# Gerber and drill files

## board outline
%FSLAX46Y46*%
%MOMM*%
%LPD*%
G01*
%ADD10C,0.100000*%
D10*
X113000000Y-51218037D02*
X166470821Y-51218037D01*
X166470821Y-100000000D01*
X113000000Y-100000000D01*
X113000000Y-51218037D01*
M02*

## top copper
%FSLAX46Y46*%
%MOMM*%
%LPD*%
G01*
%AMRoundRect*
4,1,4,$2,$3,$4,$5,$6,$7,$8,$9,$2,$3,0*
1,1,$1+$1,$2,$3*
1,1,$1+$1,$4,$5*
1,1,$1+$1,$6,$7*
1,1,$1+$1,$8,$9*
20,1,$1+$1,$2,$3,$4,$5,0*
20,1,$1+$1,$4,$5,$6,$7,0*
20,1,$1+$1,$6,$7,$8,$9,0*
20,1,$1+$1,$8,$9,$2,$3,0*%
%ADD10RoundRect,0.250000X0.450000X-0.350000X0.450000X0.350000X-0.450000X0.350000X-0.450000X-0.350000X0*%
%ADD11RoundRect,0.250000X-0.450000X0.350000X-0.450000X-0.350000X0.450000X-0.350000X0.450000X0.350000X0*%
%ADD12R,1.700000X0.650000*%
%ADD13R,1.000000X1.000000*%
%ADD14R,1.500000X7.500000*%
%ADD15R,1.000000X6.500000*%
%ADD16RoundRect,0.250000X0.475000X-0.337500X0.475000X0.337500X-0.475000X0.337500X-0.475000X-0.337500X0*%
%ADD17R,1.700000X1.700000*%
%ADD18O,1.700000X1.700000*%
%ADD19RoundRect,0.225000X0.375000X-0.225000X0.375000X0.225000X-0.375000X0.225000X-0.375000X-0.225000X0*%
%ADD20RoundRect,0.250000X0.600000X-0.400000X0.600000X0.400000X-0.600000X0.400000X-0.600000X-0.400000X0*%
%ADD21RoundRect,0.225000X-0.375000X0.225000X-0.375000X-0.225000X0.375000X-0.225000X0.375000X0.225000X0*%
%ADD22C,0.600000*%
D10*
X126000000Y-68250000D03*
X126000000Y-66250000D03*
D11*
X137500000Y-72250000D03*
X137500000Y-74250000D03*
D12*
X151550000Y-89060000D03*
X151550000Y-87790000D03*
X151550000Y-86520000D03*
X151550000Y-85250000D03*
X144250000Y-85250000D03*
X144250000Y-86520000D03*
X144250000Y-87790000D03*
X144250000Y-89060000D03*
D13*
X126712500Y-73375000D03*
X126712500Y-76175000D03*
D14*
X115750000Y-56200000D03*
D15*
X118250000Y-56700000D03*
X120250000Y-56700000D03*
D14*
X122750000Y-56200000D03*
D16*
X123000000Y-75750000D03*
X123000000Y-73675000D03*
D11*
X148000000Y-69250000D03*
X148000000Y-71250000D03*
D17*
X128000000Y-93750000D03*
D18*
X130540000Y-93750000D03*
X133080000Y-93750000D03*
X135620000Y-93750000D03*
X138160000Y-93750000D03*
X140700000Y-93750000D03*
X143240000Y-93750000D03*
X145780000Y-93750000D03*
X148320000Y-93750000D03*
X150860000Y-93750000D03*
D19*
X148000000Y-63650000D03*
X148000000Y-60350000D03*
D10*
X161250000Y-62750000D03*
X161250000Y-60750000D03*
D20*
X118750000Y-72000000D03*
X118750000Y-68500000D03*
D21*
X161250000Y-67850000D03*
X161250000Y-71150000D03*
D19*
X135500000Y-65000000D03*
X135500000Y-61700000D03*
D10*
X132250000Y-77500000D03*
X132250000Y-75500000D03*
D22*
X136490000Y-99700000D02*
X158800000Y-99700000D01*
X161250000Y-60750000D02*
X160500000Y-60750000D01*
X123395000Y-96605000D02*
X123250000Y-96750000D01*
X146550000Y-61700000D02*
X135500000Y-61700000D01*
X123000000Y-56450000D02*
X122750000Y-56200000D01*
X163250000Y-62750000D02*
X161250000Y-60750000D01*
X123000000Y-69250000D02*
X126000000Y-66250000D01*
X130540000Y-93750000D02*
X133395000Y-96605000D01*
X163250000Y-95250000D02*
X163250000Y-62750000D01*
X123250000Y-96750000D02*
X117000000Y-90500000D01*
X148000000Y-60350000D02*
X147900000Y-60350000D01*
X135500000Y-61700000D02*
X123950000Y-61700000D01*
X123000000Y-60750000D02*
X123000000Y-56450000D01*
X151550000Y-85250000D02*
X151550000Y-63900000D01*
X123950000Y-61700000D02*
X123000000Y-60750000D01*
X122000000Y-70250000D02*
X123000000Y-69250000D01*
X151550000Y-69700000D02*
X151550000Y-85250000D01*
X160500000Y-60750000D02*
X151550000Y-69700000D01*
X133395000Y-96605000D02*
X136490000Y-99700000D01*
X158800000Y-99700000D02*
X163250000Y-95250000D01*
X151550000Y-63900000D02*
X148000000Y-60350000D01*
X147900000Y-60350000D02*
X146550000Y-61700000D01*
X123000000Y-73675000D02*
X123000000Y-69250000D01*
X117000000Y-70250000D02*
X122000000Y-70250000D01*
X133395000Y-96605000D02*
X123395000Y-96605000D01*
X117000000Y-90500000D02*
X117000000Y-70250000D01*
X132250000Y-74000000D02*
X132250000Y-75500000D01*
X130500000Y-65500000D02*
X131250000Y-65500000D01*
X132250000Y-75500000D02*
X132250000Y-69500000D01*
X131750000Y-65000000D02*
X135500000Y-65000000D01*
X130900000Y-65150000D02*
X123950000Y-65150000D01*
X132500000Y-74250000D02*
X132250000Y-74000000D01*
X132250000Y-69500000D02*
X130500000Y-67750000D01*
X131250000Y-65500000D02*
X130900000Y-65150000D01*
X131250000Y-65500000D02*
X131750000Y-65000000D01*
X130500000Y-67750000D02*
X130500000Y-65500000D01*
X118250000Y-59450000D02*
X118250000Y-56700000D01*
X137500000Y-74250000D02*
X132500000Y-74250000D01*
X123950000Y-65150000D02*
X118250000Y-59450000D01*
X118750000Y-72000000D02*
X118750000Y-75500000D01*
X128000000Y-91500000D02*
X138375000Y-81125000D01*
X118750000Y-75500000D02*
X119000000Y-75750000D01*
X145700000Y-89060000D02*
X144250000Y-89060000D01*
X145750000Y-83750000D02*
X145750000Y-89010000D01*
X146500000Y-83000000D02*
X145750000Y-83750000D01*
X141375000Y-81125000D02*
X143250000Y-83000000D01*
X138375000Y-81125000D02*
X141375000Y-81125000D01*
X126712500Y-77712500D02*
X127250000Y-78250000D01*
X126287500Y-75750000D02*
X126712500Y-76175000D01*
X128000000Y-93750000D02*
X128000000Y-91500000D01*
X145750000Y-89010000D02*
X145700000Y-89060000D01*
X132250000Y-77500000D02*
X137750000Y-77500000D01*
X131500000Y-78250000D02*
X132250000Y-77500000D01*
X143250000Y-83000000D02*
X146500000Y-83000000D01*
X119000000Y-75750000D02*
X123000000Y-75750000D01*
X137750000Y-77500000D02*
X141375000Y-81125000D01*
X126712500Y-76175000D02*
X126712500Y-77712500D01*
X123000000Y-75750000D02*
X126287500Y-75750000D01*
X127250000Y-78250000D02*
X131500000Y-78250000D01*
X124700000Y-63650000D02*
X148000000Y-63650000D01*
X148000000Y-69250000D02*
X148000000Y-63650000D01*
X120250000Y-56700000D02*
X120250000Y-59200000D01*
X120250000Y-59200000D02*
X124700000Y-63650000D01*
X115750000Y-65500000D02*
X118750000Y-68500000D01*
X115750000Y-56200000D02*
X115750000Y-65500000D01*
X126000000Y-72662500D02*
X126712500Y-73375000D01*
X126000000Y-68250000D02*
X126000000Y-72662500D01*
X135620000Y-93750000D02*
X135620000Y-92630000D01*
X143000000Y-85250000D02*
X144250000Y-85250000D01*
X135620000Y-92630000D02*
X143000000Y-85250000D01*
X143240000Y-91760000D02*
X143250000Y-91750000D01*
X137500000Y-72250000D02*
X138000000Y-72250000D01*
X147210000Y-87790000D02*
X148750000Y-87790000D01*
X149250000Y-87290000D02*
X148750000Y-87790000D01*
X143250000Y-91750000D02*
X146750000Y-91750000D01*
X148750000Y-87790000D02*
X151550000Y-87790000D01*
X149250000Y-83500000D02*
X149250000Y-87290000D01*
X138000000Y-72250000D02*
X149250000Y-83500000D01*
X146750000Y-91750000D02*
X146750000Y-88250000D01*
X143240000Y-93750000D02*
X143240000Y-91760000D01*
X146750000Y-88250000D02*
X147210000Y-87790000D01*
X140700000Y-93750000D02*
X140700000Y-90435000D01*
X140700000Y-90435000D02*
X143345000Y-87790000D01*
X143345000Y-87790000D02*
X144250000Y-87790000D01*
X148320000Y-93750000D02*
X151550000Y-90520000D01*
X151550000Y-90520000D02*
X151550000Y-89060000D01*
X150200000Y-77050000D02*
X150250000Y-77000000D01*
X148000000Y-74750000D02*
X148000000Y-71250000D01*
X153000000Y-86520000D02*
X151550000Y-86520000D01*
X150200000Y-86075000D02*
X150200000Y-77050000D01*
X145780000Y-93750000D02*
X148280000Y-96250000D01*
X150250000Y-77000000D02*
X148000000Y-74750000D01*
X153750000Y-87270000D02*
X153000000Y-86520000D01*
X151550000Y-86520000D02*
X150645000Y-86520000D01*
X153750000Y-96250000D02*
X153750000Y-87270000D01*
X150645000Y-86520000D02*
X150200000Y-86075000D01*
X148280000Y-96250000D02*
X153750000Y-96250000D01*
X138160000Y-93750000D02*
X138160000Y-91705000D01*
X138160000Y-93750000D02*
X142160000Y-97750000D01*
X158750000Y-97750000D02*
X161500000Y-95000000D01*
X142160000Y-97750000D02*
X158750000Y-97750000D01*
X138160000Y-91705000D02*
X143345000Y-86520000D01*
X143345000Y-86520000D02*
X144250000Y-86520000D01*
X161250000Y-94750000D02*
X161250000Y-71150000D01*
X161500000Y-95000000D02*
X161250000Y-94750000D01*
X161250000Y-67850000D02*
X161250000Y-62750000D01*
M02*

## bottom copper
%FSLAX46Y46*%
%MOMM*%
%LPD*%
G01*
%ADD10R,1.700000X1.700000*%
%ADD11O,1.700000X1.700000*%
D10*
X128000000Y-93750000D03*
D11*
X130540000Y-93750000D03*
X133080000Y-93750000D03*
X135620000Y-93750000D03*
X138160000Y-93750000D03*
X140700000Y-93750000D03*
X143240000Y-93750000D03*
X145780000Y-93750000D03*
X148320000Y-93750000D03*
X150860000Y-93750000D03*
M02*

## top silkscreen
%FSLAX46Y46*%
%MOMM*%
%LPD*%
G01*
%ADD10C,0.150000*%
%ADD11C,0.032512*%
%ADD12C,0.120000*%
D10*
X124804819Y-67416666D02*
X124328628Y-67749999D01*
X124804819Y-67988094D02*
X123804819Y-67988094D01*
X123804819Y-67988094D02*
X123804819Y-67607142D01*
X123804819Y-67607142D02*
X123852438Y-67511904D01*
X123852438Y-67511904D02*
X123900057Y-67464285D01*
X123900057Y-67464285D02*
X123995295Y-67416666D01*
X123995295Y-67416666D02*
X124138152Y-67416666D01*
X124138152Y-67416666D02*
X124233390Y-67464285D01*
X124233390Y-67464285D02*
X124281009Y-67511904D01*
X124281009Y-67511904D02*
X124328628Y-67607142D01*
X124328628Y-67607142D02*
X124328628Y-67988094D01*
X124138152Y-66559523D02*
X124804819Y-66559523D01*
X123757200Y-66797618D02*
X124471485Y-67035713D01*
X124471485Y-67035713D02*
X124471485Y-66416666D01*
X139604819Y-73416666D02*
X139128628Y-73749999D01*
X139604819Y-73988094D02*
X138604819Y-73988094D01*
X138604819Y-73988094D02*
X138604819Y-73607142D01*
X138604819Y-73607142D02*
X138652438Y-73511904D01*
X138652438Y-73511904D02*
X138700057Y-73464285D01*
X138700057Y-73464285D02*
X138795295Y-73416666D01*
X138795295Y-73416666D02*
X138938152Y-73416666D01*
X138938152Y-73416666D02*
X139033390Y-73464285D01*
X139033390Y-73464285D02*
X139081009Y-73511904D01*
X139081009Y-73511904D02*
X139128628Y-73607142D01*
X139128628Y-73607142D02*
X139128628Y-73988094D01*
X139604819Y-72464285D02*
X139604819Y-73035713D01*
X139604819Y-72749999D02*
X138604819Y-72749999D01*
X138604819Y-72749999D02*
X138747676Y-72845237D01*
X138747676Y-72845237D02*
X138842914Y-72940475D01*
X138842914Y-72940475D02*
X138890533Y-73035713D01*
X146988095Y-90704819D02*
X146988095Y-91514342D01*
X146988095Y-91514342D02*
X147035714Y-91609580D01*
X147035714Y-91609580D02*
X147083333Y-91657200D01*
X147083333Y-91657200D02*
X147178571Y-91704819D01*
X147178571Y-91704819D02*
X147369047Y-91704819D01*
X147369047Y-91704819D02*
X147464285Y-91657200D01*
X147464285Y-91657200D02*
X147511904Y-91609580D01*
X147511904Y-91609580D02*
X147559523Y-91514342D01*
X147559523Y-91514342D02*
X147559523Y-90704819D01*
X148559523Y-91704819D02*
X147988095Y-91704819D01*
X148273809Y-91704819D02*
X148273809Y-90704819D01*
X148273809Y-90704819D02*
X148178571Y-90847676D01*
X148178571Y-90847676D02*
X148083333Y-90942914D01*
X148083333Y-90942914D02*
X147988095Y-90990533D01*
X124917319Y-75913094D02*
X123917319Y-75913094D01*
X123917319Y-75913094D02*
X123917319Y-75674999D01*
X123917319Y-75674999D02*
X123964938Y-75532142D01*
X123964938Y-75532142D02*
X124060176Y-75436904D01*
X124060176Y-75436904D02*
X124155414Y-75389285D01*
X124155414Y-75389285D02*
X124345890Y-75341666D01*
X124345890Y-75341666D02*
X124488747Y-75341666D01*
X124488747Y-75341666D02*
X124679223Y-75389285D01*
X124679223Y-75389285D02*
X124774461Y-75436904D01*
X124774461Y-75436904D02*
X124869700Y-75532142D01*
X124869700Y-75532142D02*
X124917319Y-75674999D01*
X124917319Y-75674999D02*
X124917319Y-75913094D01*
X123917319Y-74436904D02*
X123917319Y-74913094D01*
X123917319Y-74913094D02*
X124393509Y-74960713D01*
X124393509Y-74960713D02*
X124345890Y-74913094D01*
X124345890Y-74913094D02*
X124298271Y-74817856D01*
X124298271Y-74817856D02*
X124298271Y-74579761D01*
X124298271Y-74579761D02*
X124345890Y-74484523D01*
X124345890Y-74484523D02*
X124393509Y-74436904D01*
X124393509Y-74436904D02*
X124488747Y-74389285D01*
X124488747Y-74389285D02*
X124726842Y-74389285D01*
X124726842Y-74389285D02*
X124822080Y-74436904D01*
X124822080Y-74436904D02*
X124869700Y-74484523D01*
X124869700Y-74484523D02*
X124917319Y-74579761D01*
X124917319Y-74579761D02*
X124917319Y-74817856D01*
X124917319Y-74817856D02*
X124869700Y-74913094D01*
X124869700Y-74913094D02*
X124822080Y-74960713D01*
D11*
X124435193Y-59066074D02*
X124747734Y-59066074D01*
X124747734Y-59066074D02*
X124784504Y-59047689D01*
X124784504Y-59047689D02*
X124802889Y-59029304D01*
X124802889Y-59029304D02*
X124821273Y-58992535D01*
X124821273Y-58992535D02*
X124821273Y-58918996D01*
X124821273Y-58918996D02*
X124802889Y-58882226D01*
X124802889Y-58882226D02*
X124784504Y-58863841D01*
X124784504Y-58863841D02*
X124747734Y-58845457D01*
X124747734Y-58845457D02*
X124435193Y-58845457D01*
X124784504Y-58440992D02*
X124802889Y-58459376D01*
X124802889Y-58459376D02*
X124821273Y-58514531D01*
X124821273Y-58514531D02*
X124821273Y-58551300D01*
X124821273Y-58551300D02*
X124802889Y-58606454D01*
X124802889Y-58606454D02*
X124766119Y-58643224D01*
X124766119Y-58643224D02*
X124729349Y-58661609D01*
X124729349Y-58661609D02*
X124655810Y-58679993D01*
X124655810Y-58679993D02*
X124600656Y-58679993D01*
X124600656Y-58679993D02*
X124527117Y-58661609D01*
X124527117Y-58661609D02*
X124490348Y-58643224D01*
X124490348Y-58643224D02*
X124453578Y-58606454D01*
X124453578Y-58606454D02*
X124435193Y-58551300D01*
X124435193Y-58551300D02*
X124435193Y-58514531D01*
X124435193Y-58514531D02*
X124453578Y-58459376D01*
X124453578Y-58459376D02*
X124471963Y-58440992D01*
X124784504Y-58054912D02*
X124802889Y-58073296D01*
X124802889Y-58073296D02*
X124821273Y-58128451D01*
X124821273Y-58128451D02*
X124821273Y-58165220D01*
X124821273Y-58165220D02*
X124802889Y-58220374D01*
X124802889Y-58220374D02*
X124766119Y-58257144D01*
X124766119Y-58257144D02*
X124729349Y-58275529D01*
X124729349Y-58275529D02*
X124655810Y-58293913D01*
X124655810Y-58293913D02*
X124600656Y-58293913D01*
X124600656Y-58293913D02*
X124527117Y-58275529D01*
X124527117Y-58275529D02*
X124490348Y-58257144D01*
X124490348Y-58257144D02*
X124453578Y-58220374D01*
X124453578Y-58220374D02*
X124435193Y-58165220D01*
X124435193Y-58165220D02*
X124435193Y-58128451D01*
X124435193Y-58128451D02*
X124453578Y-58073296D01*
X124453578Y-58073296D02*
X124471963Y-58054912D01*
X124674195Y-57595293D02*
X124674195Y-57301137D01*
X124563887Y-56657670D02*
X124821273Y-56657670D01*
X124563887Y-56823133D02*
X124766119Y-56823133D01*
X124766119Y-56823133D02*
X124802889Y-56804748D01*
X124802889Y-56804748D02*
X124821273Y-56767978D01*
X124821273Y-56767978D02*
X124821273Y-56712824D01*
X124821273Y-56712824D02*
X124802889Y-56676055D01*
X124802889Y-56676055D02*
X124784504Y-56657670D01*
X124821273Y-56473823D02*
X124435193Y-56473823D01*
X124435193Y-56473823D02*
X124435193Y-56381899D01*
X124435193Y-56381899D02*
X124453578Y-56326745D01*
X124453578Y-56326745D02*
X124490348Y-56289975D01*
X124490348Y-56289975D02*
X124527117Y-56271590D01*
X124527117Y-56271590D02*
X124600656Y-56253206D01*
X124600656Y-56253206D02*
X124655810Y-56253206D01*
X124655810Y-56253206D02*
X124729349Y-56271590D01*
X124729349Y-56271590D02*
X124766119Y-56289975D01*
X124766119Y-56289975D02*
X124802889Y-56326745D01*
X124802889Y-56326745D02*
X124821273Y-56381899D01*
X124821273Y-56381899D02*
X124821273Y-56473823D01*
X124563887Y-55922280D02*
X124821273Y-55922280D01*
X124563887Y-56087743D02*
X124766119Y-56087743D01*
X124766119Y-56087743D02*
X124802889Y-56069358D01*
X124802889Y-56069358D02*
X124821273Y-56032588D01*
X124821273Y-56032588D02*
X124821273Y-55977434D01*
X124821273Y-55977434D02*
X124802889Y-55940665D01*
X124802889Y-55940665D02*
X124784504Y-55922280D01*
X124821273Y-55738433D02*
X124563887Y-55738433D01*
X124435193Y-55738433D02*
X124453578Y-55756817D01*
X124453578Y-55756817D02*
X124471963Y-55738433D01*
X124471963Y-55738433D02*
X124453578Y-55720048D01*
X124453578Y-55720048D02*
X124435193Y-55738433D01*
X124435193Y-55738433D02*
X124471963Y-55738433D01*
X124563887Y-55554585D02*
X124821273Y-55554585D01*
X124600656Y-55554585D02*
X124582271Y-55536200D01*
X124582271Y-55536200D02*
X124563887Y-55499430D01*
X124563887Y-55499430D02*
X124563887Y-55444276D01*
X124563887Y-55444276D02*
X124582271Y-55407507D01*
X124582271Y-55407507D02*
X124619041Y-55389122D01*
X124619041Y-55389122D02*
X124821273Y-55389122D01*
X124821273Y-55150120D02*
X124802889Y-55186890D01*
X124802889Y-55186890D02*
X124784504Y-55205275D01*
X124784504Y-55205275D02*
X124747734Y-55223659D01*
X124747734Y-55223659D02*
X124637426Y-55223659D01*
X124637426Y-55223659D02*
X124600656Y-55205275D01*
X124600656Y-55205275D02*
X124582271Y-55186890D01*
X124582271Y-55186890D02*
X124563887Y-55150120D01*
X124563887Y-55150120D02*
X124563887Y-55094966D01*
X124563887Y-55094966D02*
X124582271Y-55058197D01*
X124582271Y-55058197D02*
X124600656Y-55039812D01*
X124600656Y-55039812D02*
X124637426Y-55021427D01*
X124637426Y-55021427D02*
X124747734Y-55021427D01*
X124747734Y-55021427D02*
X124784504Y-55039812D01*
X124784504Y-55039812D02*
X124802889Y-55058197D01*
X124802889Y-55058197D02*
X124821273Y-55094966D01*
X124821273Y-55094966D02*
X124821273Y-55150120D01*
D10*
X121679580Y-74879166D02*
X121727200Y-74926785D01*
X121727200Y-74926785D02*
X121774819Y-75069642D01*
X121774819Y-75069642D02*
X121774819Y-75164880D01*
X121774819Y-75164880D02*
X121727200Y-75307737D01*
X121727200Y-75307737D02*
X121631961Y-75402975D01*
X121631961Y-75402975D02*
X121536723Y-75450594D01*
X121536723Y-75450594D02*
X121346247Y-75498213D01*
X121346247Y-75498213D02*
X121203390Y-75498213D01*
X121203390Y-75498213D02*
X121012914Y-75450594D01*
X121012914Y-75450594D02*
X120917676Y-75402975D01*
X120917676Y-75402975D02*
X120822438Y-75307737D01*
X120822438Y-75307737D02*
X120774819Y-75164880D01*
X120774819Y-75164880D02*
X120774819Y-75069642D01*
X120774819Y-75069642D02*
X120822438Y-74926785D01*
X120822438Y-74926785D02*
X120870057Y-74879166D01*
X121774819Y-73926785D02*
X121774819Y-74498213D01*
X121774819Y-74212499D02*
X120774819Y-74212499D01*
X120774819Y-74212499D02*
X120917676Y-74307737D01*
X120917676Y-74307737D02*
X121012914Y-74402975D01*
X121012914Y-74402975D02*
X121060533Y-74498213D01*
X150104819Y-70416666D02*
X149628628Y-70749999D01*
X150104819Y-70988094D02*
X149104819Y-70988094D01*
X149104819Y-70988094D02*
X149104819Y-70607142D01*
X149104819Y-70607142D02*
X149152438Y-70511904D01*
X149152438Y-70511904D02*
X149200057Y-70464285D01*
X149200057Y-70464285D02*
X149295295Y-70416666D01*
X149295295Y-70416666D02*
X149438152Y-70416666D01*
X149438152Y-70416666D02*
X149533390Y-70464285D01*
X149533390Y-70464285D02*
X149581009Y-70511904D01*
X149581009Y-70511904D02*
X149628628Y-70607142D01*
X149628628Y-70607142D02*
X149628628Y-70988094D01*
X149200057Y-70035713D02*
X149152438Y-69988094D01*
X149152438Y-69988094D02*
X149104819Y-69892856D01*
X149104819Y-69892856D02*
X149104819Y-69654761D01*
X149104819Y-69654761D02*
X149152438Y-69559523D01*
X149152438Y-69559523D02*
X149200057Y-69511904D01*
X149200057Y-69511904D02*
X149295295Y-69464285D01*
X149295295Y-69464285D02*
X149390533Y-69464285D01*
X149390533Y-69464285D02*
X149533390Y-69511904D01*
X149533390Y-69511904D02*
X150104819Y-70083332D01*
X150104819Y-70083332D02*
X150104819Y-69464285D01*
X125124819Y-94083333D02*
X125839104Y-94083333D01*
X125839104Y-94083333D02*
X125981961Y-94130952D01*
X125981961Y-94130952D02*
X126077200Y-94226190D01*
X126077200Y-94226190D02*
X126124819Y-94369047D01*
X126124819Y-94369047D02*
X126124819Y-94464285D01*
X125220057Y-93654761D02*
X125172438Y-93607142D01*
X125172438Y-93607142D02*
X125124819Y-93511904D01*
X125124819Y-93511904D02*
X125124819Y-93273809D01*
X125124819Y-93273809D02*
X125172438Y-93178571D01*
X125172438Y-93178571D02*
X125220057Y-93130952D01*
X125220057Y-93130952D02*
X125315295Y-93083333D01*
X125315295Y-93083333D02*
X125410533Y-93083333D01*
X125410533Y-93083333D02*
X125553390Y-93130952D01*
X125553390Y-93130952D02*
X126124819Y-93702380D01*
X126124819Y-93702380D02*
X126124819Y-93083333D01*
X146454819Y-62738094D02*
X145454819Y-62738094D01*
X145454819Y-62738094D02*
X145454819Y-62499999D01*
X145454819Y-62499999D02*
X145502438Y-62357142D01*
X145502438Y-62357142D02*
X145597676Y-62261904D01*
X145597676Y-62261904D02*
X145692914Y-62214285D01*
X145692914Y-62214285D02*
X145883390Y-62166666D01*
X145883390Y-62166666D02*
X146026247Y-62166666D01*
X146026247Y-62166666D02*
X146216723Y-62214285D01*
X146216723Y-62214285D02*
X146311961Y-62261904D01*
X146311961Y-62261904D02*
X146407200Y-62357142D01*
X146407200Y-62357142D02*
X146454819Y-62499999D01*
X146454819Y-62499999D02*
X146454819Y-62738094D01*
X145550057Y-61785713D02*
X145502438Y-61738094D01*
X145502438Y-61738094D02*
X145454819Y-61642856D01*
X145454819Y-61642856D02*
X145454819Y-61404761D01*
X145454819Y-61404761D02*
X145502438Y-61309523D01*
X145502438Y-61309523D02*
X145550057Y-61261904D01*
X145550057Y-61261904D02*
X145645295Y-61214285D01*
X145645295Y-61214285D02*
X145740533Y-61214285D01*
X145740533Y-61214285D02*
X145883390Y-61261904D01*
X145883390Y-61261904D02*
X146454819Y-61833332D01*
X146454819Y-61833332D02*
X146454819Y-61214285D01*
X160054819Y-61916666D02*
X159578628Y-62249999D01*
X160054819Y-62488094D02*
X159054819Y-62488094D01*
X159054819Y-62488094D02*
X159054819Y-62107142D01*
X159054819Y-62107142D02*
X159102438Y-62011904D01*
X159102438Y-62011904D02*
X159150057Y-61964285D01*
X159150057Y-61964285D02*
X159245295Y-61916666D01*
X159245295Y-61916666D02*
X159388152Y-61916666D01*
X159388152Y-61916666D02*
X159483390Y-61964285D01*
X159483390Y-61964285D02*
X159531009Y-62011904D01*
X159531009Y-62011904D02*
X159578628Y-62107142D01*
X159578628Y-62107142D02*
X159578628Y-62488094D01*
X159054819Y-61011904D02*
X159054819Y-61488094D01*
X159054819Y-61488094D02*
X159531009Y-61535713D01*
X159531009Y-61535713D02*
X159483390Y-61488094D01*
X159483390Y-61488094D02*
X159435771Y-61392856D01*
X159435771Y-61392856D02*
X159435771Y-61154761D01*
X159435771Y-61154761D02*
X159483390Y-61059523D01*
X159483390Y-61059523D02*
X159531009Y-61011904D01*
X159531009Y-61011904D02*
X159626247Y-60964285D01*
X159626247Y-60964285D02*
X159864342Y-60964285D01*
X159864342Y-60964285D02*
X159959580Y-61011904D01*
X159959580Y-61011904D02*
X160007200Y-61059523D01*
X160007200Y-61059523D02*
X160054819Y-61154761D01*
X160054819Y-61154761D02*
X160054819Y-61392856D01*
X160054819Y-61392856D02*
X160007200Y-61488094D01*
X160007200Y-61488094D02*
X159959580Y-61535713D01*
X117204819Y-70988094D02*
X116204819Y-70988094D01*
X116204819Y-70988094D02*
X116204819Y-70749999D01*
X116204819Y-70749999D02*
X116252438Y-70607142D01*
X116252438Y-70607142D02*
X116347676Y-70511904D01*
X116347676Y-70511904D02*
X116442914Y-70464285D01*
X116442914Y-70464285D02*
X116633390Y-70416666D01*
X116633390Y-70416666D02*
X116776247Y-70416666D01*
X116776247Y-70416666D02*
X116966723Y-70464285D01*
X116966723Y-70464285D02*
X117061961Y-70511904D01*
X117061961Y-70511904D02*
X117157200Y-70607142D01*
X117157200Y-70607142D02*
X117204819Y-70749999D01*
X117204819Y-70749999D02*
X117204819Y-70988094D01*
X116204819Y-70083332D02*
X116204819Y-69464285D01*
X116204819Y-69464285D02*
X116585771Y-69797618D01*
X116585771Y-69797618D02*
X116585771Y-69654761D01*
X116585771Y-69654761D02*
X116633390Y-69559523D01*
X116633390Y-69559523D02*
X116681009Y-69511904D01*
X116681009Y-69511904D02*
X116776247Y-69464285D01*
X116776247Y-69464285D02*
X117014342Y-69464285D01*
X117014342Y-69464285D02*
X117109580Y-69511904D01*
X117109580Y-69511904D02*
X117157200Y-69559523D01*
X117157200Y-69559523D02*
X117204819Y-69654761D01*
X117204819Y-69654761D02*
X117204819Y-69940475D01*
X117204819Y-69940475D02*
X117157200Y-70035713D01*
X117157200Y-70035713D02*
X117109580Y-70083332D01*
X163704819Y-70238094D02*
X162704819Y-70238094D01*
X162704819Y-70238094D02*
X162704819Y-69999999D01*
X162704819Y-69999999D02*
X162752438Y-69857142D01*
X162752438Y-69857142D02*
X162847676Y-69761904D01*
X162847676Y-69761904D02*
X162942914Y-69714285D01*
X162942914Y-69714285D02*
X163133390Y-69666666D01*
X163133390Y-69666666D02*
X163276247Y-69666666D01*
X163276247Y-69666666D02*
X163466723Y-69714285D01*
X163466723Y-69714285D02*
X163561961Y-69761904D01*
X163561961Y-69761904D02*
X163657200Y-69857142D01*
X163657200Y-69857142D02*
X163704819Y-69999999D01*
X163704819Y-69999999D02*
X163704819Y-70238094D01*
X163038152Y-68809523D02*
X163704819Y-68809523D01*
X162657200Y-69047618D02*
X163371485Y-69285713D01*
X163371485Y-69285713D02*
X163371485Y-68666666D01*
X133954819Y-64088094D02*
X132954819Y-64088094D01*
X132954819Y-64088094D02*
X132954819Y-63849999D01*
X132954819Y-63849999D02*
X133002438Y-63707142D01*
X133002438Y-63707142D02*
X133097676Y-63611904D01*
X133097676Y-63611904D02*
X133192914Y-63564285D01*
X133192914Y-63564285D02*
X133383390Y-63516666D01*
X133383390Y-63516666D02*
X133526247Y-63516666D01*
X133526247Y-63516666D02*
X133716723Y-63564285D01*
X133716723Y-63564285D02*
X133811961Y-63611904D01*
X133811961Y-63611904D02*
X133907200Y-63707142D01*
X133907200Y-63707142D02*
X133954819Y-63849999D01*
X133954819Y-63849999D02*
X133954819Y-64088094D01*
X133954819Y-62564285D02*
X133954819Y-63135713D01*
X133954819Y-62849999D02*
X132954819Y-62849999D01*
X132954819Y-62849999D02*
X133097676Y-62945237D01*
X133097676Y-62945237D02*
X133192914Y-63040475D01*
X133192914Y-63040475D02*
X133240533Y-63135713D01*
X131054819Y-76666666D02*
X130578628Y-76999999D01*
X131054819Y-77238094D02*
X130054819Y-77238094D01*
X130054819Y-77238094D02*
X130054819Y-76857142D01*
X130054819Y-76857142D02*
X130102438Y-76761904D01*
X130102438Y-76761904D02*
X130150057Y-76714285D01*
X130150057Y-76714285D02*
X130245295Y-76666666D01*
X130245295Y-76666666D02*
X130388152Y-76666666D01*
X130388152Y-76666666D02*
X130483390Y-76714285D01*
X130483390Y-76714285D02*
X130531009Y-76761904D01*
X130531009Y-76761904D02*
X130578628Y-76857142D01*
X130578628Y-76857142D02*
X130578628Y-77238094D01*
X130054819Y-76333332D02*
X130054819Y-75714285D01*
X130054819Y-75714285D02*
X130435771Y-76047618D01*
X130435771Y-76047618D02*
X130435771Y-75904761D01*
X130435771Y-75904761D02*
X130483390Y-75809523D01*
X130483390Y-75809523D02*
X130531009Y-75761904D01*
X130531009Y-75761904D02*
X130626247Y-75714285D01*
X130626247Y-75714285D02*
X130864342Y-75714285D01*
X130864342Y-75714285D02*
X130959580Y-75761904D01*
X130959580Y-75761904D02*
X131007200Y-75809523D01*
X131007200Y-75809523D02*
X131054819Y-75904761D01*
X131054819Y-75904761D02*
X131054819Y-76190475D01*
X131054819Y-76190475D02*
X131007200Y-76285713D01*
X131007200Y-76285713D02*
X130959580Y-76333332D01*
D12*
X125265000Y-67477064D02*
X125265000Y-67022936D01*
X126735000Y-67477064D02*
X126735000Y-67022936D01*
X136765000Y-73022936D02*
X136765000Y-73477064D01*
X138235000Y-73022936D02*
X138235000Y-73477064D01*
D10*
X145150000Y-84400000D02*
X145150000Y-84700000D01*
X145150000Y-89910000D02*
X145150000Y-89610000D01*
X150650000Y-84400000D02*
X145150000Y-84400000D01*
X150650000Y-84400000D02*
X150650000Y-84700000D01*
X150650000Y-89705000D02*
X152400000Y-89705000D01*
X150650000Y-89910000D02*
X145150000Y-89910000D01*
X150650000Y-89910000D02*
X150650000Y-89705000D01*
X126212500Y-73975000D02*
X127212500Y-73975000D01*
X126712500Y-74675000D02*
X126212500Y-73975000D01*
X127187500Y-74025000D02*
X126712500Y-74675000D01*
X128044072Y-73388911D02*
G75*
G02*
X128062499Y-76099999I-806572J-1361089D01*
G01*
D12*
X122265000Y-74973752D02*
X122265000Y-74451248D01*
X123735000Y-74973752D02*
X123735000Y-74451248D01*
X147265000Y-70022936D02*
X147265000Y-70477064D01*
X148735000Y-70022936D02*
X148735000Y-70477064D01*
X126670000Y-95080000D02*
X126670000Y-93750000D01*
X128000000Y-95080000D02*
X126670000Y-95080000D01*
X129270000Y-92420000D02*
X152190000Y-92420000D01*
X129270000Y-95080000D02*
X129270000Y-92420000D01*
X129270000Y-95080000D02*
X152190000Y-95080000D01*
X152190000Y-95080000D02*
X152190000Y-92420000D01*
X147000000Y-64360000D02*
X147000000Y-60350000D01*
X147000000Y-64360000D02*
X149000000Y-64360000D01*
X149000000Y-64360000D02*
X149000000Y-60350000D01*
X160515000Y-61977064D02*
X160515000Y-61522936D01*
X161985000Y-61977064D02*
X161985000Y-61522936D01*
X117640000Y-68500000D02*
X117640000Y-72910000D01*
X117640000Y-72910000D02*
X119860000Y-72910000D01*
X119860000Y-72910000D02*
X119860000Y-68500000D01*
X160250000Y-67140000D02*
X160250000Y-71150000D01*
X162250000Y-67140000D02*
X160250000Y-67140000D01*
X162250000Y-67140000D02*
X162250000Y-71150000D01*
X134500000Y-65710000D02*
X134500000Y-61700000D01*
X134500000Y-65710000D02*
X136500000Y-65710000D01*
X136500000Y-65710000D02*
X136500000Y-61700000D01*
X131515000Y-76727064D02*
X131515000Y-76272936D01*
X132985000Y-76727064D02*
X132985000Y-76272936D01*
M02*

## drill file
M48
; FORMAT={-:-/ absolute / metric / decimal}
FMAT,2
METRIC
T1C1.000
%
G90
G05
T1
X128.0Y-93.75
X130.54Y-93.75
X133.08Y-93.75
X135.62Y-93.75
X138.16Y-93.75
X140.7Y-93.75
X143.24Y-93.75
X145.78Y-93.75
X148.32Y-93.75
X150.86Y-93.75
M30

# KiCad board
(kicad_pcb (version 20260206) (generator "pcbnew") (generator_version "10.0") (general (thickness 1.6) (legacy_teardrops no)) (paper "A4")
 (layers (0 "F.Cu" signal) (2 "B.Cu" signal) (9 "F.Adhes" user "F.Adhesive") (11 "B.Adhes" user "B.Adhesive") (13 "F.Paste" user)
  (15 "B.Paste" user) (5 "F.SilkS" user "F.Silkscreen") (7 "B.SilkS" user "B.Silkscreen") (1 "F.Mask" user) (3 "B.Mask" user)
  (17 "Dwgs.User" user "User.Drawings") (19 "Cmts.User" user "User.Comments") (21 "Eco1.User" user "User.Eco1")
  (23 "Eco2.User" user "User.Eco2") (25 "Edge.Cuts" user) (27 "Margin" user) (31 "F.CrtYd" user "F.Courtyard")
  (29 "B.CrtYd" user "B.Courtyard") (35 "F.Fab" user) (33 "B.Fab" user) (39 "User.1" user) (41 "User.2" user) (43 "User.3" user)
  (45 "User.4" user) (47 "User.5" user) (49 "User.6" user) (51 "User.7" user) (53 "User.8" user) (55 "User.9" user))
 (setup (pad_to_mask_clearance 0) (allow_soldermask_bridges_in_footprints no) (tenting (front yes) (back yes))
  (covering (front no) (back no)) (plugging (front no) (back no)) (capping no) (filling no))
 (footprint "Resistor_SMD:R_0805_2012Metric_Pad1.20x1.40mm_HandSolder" (layer "F.Cu") (at 126 67.25 90)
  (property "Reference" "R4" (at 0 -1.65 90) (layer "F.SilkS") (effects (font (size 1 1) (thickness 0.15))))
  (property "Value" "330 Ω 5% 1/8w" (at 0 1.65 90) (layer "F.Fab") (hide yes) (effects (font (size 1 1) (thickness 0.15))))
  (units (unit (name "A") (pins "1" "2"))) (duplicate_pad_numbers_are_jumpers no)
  (fp_line (start -0.227064 -0.735) (end 0.227064 -0.735) (stroke (width 0.12) (type solid)) (layer "F.SilkS"))
  (fp_line (start -0.227064 0.735) (end 0.227064 0.735) (stroke (width 0.12) (type solid)) (layer "F.SilkS"))
  (pad "1" smd roundrect (at -1 0 90) (size 1.2 1.4) (layers "F.Cu" "F.Mask" "F.Paste") (roundrect_rratio 0.208333) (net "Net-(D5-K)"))
  (pad "2" smd roundrect (at 1 0 90) (size 1.2 1.4) (layers "F.Cu" "F.Mask" "F.Paste") (roundrect_rratio 0.208333) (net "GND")))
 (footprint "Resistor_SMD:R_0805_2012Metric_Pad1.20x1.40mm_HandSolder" (layer "F.Cu") (at 137.5 73.25 -90)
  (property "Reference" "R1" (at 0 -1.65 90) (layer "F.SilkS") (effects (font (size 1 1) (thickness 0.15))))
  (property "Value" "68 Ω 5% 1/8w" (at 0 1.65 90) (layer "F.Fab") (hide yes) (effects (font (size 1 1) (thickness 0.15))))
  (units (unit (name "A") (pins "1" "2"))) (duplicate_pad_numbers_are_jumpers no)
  (fp_line (start -0.227064 0.735) (end 0.227064 0.735) (stroke (width 0.12) (type solid)) (layer "F.SilkS"))
  (fp_line (start -0.227064 -0.735) (end 0.227064 -0.735) (stroke (width 0.12) (type solid)) (layer "F.SilkS"))
  (pad "1" smd roundrect (at -1 0 270) (size 1.2 1.4) (layers "F.Cu" "F.Mask" "F.Paste") (roundrect_rratio 0.208333) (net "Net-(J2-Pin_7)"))
  (pad "2" smd roundrect (at 1 0 270) (size 1.2 1.4) (layers "F.Cu" "F.Mask" "F.Paste") (roundrect_rratio 0.208333) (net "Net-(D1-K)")))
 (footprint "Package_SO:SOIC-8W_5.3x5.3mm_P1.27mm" (layer "F.Cu") (at 147.9 87.155 180)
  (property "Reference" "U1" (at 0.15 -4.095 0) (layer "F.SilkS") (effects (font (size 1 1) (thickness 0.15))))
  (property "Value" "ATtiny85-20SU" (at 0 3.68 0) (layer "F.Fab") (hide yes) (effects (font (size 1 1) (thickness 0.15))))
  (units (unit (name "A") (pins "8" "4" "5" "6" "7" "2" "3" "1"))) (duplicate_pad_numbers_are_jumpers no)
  (fp_line (start 2.75 2.755) (end 2.75 2.455) (stroke (width 0.15) (type solid)) (layer "F.SilkS"))
  (fp_line (start 2.75 -2.755) (end 2.75 -2.455) (stroke (width 0.15) (type solid)) (layer "F.SilkS"))
  (fp_line (start -2.75 2.755) (end 2.75 2.755) (stroke (width 0.15) (type solid)) (layer "F.SilkS"))
  (fp_line (start -2.75 2.755) (end -2.75 2.455) (stroke (width 0.15) (type solid)) (layer "F.SilkS"))
  (fp_line (start -2.75 -2.55) (end -4.5 -2.55) (stroke (width 0.15) (type solid)) (layer "F.SilkS"))
  (fp_line (start -2.75 -2.755) (end 2.75 -2.755) (stroke (width 0.15) (type solid)) (layer "F.SilkS"))
  (fp_line (start -2.75 -2.755) (end -2.75 -2.55) (stroke (width 0.15) (type solid)) (layer "F.SilkS"))
  (pad "1" smd rect (at -3.65 -1.905 180) (size 1.7 0.65) (layers "F.Cu" "F.Mask" "F.Paste") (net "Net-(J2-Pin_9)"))
  (pad "2" smd rect (at -3.65 -0.635 180) (size 1.7 0.65) (layers "F.Cu" "F.Mask" "F.Paste") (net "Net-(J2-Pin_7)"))
  (pad "3" smd rect (at -3.65 0.635 180) (size 1.7 0.65) (layers "F.Cu" "F.Mask" "F.Paste") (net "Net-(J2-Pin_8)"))
  (pad "4" smd rect (at -3.65 1.905 180) (size 1.7 0.65) (layers "F.Cu" "F.Mask" "F.Paste") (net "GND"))
  (pad "5" smd rect (at 3.65 1.905 180) (size 1.7 0.65) (layers "F.Cu" "F.Mask" "F.Paste") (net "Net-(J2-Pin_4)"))
  (pad "6" smd rect (at 3.65 0.635 180) (size 1.7 0.65) (layers "F.Cu" "F.Mask" "F.Paste") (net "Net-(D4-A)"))
  (pad "7" smd rect (at 3.65 -0.635 180) (size 1.7 0.65) (layers "F.Cu" "F.Mask" "F.Paste") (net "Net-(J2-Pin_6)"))
  (pad "8" smd rect (at 3.65 -1.905 180) (size 1.7 0.65) (layers "F.Cu" "F.Mask" "F.Paste") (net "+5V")))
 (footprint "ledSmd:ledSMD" (layer "F.Cu") (at 126.7125 75.175 -90)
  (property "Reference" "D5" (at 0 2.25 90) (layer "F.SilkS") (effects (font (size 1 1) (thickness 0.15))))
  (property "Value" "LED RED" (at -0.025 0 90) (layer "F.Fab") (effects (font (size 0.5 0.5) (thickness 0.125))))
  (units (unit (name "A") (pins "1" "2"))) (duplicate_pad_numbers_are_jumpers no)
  (fp_line (start -1.2 0.5) (end -1.2 -0.5) (stroke (width 0.15) (type solid)) (layer "F.SilkS"))
  (fp_line (start -0.5 0) (end -1.2 0.5) (stroke (width 0.15) (type solid)) (layer "F.SilkS"))
  (fp_line (start -1.15 -0.475) (end -0.5 0) (stroke (width 0.15) (type solid)) (layer "F.SilkS"))
  (fp_arc (start -1.786089 -1.331572) (mid -0.435753 -2.107089) (end 0.924999 -1.349999) (stroke (width 0.15) (type solid))
   (layer "F.SilkS"))
  (pad "1" smd rect (at -1.8 0 270) (size 1 1) (layers "F.Cu" "F.Mask" "F.Paste") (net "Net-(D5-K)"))
  (pad "2" smd rect (at 1 0 270) (size 1 1) (layers "F.Cu" "F.Mask" "F.Paste") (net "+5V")))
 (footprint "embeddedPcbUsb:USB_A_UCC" (layer "F.Cu") (at 119.25 56.4 -90)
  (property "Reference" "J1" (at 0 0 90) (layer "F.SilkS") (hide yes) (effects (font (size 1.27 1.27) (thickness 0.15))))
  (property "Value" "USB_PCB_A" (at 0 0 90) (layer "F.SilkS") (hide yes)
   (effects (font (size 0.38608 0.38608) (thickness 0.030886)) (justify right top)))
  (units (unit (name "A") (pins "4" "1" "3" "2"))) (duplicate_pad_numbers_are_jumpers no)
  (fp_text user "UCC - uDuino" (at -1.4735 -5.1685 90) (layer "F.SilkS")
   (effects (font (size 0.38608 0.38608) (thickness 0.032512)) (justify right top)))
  (pad "1" smd rect (at -0.2 3.5 270) (size 7.5 1.5) (layers "F.Cu" "F.Mask" "F.Paste") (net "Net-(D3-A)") (solder_mask_margin 0.1016))
  (pad "2" smd rect (at 0.3 1 270) (size 6.5 1) (layers "F.Cu" "F.Mask" "F.Paste") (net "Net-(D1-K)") (solder_mask_margin 0.1016))
  (pad "3" smd rect (at 0.3 -1 270) (size 6.5 1) (layers "F.Cu" "F.Mask" "F.Paste") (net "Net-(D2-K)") (solder_mask_margin 0.1016))
  (pad "4" smd rect (at -0.2 -3.5 270) (size 7.5 1.5) (layers "F.Cu" "F.Mask" "F.Paste") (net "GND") (solder_mask_margin 0.1016)))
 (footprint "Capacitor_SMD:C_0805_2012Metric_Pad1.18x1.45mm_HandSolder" (layer "F.Cu") (at 123 74.7125 90)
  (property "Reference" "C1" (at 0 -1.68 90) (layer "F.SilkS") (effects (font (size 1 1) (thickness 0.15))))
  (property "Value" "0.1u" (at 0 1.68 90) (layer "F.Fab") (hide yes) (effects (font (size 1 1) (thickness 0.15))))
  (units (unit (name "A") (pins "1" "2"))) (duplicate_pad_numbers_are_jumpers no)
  (fp_line (start -0.261252 -0.735) (end 0.261252 -0.735) (stroke (width 0.12) (type solid)) (layer "F.SilkS"))
  (fp_line (start -0.261252 0.735) (end 0.261252 0.735) (stroke (width 0.12) (type solid)) (layer "F.SilkS"))
  (pad "1" smd roundrect (at -1.0375 0 90) (size 1.175 1.45) (layers "F.Cu" "F.Mask" "F.Paste") (roundrect_rratio 0.212766) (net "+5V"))
  (pad "2" smd roundrect (at 1.0375 0 90) (size 1.175 1.45) (layers "F.Cu" "F.Mask" "F.Paste") (roundrect_rratio 0.212766) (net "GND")))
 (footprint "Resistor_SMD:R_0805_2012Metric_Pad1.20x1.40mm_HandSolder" (layer "F.Cu") (at 148 70.25 -90)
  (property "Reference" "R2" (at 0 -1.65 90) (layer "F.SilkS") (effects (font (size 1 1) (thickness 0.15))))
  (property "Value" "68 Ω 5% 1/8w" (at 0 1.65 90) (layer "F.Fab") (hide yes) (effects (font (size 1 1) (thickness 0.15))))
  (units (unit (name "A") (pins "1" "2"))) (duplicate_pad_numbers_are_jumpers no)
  (fp_line (start -0.227064 0.735) (end 0.227064 0.735) (stroke (width 0.12) (type solid)) (layer "F.SilkS"))
  (fp_line (start -0.227064 -0.735) (end 0.227064 -0.735) (stroke (width 0.12) (type solid)) (layer "F.SilkS"))
  (pad "1" smd roundrect (at -1 0 270) (size 1.2 1.4) (layers "F.Cu" "F.Mask" "F.Paste") (roundrect_rratio 0.208333) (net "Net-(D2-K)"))
  (pad "2" smd roundrect (at 1 0 270) (size 1.2 1.4) (layers "F.Cu" "F.Mask" "F.Paste") (roundrect_rratio 0.208333) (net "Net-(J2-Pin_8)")))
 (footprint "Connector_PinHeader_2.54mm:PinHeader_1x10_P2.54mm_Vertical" (layer "F.Cu") (at 128 93.75 90)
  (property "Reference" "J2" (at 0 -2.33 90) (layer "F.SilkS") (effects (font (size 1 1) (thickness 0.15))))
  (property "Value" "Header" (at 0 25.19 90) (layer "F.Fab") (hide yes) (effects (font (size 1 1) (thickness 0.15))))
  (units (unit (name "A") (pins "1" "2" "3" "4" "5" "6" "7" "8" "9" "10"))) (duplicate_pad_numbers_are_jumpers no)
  (fp_line (start -1.33 -1.33) (end 0 -1.33) (stroke (width 0.12) (type solid)) (layer "F.SilkS"))
  (fp_line (start -1.33 0) (end -1.33 -1.33) (stroke (width 0.12) (type solid)) (layer "F.SilkS"))
  (fp_line (start 1.33 1.27) (end 1.33 24.19) (stroke (width 0.12) (type solid)) (layer "F.SilkS"))
  (fp_line (start -1.33 1.27) (end 1.33 1.27) (stroke (width 0.12) (type solid)) (layer "F.SilkS"))
  (fp_line (start -1.33 1.27) (end -1.33 24.19) (stroke (width 0.12) (type solid)) (layer "F.SilkS"))
  (fp_line (start -1.33 24.19) (end 1.33 24.19) (stroke (width 0.12) (type solid)) (layer "F.SilkS"))
  (pad "1" thru_hole rect (at 0 0 90) (size 1.7 1.7) (drill 1) (layers "*.Cu" "*.Mask") (remove_unused_layers no) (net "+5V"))
  (pad "2" thru_hole oval (at 0 2.54 90) (size 1.7 1.7) (drill 1) (layers "*.Cu" "*.Mask") (remove_unused_layers no) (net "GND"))
  (pad "3" thru_hole oval (at 0 5.08 90) (size 1.7 1.7) (drill 1) (layers "*.Cu" "*.Mask") (remove_unused_layers no)
   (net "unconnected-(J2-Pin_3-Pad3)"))
  (pad "4" thru_hole oval (at 0 7.62 90) (size 1.7 1.7) (drill 1) (layers "*.Cu" "*.Mask") (remove_unused_layers no) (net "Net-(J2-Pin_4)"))
  (pad "5" thru_hole oval (at 0 10.16 90) (size 1.7 1.7) (drill 1) (layers "*.Cu" "*.Mask") (remove_unused_layers no) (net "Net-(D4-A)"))
  (pad "6" thru_hole oval (at 0 12.7 90) (size 1.7 1.7) (drill 1) (layers "*.Cu" "*.Mask") (remove_unused_layers no) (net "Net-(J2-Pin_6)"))
  (pad "7" thru_hole oval (at 0 15.24 90) (size 1.7 1.7) (drill 1) (layers "*.Cu" "*.Mask") (remove_unused_layers no) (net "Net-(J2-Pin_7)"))
  (pad "8" thru_hole oval (at 0 17.78 90) (size 1.7 1.7) (drill 1) (layers "*.Cu" "*.Mask") (remove_unused_layers no) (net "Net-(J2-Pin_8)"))
  (pad "9" thru_hole oval (at 0 20.32 90) (size 1.7 1.7) (drill 1) (layers "*.Cu" "*.Mask") (remove_unused_layers no) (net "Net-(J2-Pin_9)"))
  (pad "10" thru_hole oval (at 0 22.86 90) (size 1.7 1.7) (drill 1) (layers "*.Cu" "*.Mask") (remove_unused_layers no)
   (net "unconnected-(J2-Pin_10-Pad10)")))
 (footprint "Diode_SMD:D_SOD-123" (layer "F.Cu") (at 148 62 90)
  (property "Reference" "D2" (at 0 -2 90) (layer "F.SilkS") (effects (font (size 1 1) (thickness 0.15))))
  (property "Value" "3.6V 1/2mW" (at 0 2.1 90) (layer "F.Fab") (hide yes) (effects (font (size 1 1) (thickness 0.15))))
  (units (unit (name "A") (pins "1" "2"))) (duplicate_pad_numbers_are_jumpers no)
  (fp_line (start -2.36 -1) (end 1.65 -1) (stroke (width 0.12) (type solid)) (layer "F.SilkS"))
  (fp_line (start -2.36 -1) (end -2.36 1) (stroke (width 0.12) (type solid)) (layer "F.SilkS"))
  (fp_line (start -2.36 1) (end 1.65 1) (stroke (width 0.12) (type solid)) (layer "F.SilkS"))
  (pad "1" smd roundrect (at -1.65 0 90) (size 0.9 1.2) (layers "F.Cu" "F.Mask" "F.Paste") (roundrect_rratio 0.25) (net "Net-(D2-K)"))
  (pad "2" smd roundrect (at 1.65 0 90) (size 0.9 1.2) (layers "F.Cu" "F.Mask" "F.Paste") (roundrect_rratio 0.25) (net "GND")))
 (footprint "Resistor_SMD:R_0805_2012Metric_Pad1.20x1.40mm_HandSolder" (layer "F.Cu") (at 161.25 61.75 90)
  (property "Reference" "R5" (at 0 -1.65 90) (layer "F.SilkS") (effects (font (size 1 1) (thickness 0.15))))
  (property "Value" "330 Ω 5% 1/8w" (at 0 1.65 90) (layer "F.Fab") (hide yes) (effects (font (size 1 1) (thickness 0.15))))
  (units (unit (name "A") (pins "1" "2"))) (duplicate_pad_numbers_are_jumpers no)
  (fp_line (start -0.227064 -0.735) (end 0.227064 -0.735) (stroke (width 0.12) (type solid)) (layer "F.SilkS"))
  (fp_line (start -0.227064 0.735) (end 0.227064 0.735) (stroke (width 0.12) (type solid)) (layer "F.SilkS"))
  (pad "1" smd roundrect (at -1 0 90) (size 1.2 1.4) (layers "F.Cu" "F.Mask" "F.Paste") (roundrect_rratio 0.208333) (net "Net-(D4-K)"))
  (pad "2" smd roundrect (at 1 0 90) (size 1.2 1.4) (layers "F.Cu" "F.Mask" "F.Paste") (roundrect_rratio 0.208333) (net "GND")))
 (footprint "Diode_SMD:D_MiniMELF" (layer "F.Cu") (at 118.75 70.25 90)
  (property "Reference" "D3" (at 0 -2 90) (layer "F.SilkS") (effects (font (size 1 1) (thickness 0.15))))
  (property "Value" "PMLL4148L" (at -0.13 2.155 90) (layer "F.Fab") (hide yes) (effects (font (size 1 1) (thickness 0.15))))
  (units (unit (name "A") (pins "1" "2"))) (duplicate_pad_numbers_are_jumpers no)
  (fp_line (start 1.75 -1.11) (end -2.66 -1.11) (stroke (width 0.12) (type solid)) (layer "F.SilkS"))
  (fp_line (start -2.66 -1.11) (end -2.66 1.11) (stroke (width 0.12) (type solid)) (layer "F.SilkS"))
  (fp_line (start -2.66 1.11) (end 1.75 1.11) (stroke (width 0.12) (type solid)) (layer "F.SilkS"))
  (pad "1" smd roundrect (at -1.75 0 90) (size 1.3 1.7) (layers "F.Cu" "F.Mask" "F.Paste") (roundrect_rratio 0.1923076923) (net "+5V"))
  (pad "2" smd roundrect (at 1.75 0 90) (size 1.3 1.7) (layers "F.Cu" "F.Mask" "F.Paste") (roundrect_rratio 0.1923076923) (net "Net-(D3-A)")))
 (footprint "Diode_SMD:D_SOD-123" (layer "F.Cu") (at 161.25 69.5 -90)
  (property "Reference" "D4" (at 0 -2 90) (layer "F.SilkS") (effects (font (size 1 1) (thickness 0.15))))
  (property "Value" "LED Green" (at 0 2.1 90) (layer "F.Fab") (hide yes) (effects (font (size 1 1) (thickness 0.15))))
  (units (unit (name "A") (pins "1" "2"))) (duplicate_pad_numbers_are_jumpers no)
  (fp_line (start -2.36 1) (end 1.65 1) (stroke (width 0.12) (type solid)) (layer "F.SilkS"))
  (fp_line (start -2.36 -1) (end -2.36 1) (stroke (width 0.12) (type solid)) (layer "F.SilkS"))
  (fp_line (start -2.36 -1) (end 1.65 -1) (stroke (width 0.12) (type solid)) (layer "F.SilkS"))
  (pad "1" smd roundrect (at -1.65 0 270) (size 0.9 1.2) (layers "F.Cu" "F.Mask" "F.Paste") (roundrect_rratio 0.25) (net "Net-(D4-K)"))
  (pad "2" smd roundrect (at 1.65 0 270) (size 0.9 1.2) (layers "F.Cu" "F.Mask" "F.Paste") (roundrect_rratio 0.25) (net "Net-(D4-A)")))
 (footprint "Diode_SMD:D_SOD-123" (layer "F.Cu") (at 135.5 63.35 90)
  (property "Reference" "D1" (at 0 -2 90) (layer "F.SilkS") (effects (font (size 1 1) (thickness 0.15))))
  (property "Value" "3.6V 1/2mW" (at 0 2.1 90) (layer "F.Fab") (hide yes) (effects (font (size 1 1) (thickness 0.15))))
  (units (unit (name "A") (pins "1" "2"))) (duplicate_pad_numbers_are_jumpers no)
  (fp_line (start -2.36 -1) (end 1.65 -1) (stroke (width 0.12) (type solid)) (layer "F.SilkS"))
  (fp_line (start -2.36 -1) (end -2.36 1) (stroke (width 0.12) (type solid)) (layer "F.SilkS"))
  (fp_line (start -2.36 1) (end 1.65 1) (stroke (width 0.12) (type solid)) (layer "F.SilkS"))
  (pad "1" smd roundrect (at -1.65 0 90) (size 0.9 1.2) (layers "F.Cu" "F.Mask" "F.Paste") (roundrect_rratio 0.25) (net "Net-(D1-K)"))
  (pad "2" smd roundrect (at 1.65 0 90) (size 0.9 1.2) (layers "F.Cu" "F.Mask" "F.Paste") (roundrect_rratio 0.25) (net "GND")))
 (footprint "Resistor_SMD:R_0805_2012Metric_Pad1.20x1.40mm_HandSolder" (layer "F.Cu") (at 132.25 76.5 90)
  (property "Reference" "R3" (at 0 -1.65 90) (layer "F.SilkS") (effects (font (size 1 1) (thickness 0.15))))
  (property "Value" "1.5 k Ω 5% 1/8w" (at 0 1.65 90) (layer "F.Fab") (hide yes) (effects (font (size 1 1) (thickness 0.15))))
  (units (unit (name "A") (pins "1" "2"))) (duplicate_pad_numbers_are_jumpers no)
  (fp_line (start -0.227064 -0.735) (end 0.227064 -0.735) (stroke (width 0.12) (type solid)) (layer "F.SilkS"))
  (fp_line (start -0.227064 0.735) (end 0.227064 0.735) (stroke (width 0.12) (type solid)) (layer "F.SilkS"))
  (pad "1" smd roundrect (at -1 0 90) (size 1.2 1.4) (layers "F.Cu" "F.Mask" "F.Paste") (roundrect_rratio 0.208333) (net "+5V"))
  (pad "2" smd roundrect (at 1 0 90) (size 1.2 1.4) (layers "F.Cu" "F.Mask" "F.Paste") (roundrect_rratio 0.208333) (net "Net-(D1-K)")))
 (gr_rect (start 113 51.218037) (end 166.470821 100) (stroke (width 0.1) (type default)) (fill no) (layer "Edge.Cuts"))
 (segment (start 136.49 99.7) (end 158.8 99.7) (width 0.6) (layer "F.Cu") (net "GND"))
 (segment (start 161.25 60.75) (end 160.5 60.75) (width 0.6) (layer "F.Cu") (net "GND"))
 (segment (start 123.395 96.605) (end 123.25 96.75) (width 0.6) (layer "F.Cu") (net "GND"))
 (segment (start 146.55 61.7) (end 135.5 61.7) (width 0.6) (layer "F.Cu") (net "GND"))
 (segment (start 123 56.45) (end 122.75 56.2) (width 0.6) (layer "F.Cu") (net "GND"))
 (segment (start 163.25 62.75) (end 161.25 60.75) (width 0.6) (layer "F.Cu") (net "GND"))
 (segment (start 123 69.25) (end 126 66.25) (width 0.6) (layer "F.Cu") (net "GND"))
 (segment (start 130.54 93.75) (end 133.395 96.605) (width 0.6) (layer "F.Cu") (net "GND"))
 (segment (start 163.25 95.25) (end 163.25 62.75) (width 0.6) (layer "F.Cu") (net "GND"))
 (segment (start 123.25 96.75) (end 117 90.5) (width 0.6) (layer "F.Cu") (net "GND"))
 (segment (start 148 60.35) (end 147.9 60.35) (width 0.6) (layer "F.Cu") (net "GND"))
 (segment (start 135.5 61.7) (end 123.95 61.7) (width 0.6) (layer "F.Cu") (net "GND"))
 (segment (start 123 60.75) (end 123 56.45) (width 0.6) (layer "F.Cu") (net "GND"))
 (segment (start 151.55 85.25) (end 151.55 63.9) (width 0.6) (layer "F.Cu") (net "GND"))
 (segment (start 123.95 61.7) (end 123 60.75) (width 0.6) (layer "F.Cu") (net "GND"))
 (segment (start 122 70.25) (end 123 69.25) (width 0.6) (layer "F.Cu") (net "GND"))
 (segment (start 151.55 69.7) (end 151.55 85.25) (width 0.6) (layer "F.Cu") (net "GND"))
 (segment (start 160.5 60.75) (end 151.55 69.7) (width 0.6) (layer "F.Cu") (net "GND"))
 (segment (start 133.395 96.605) (end 136.49 99.7) (width 0.6) (layer "F.Cu") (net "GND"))
 (segment (start 158.8 99.7) (end 163.25 95.25) (width 0.6) (layer "F.Cu") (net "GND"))
 (segment (start 151.55 63.9) (end 148 60.35) (width 0.6) (layer "F.Cu") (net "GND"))
 (segment (start 147.9 60.35) (end 146.55 61.7) (width 0.6) (layer "F.Cu") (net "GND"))
 (segment (start 123 73.675) (end 123 69.25) (width 0.6) (layer "F.Cu") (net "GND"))
 (segment (start 117 70.25) (end 122 70.25) (width 0.6) (layer "F.Cu") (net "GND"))
 (segment (start 133.395 96.605) (end 123.395 96.605) (width 0.6) (layer "F.Cu") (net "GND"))
 (segment (start 117 90.5) (end 117 70.25) (width 0.6) (layer "F.Cu") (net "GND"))
 (segment (start 132.25 74) (end 132.25 75.5) (width 0.6) (layer "F.Cu") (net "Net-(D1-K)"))
 (segment (start 130.5 65.5) (end 131.25 65.5) (width 0.6) (layer "F.Cu") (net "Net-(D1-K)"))
 (segment (start 132.25 75.5) (end 132.25 69.5) (width 0.6) (layer "F.Cu") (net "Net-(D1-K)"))
 (segment (start 131.75 65) (end 135.5 65) (width 0.6) (layer "F.Cu") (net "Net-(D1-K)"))
 (segment (start 130.9 65.15) (end 123.95 65.15) (width 0.6) (layer "F.Cu") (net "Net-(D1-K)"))
 (segment (start 132.5 74.25) (end 132.25 74) (width 0.6) (layer "F.Cu") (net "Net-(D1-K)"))
 (segment (start 132.25 69.5) (end 130.5 67.75) (width 0.6) (layer "F.Cu") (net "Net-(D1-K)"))
 (segment (start 131.25 65.5) (end 130.9 65.15) (width 0.6) (layer "F.Cu") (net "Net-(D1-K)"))
 (segment (start 131.25 65.5) (end 131.75 65) (width 0.6) (layer "F.Cu") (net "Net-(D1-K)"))
 (segment (start 130.5 67.75) (end 130.5 65.5) (width 0.6) (layer "F.Cu") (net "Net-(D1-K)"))
 (segment (start 118.25 59.45) (end 118.25 56.7) (width 0.6) (layer "F.Cu") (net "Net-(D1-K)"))
 (segment (start 137.5 74.25) (end 132.5 74.25) (width 0.6) (layer "F.Cu") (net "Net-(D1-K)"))
 (segment (start 123.95 65.15) (end 118.25 59.45) (width 0.6) (layer "F.Cu") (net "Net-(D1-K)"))
 (segment (start 118.75 72) (end 118.75 75.5) (width 0.6) (layer "F.Cu") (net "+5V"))
 (segment (start 128 91.5) (end 138.375 81.125) (width 0.6) (layer "F.Cu") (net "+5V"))
 (segment (start 118.75 75.5) (end 119 75.75) (width 0.6) (layer "F.Cu") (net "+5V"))
 (segment (start 145.7 89.06) (end 144.25 89.06) (width 0.6) (layer "F.Cu") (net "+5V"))
 (segment (start 145.75 83.75) (end 145.75 89.01) (width 0.6) (layer "F.Cu") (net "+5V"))
 (segment (start 146.5 83) (end 145.75 83.75) (width 0.6) (layer "F.Cu") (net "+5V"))
 (segment (start 141.375 81.125) (end 143.25 83) (width 0.6) (layer "F.Cu") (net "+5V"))
 (segment (start 138.375 81.125) (end 141.375 81.125) (width 0.6) (layer "F.Cu") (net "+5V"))
 (segment (start 126.7125 77.7125) (end 127.25 78.25) (width 0.6) (layer "F.Cu") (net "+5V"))
 (segment (start 126.2875 75.75) (end 126.7125 76.175) (width 0.6) (layer "F.Cu") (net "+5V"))
 (segment (start 128 93.75) (end 128 91.5) (width 0.6) (layer "F.Cu") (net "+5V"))
 (segment (start 145.75 89.01) (end 145.7 89.06) (width 0.6) (layer "F.Cu") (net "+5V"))
 (segment (start 132.25 77.5) (end 137.75 77.5) (width 0.6) (layer "F.Cu") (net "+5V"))
 (segment (start 131.5 78.25) (end 132.25 77.5) (width 0.6) (layer "F.Cu") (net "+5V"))
 (segment (start 143.25 83) (end 146.5 83) (width 0.6) (layer "F.Cu") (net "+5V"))
 (segment (start 119 75.75) (end 123 75.75) (width 0.6) (layer "F.Cu") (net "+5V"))
 (segment (start 137.75 77.5) (end 141.375 81.125) (width 0.6) (layer "F.Cu") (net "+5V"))
 (segment (start 126.7125 76.175) (end 126.7125 77.7125) (width 0.6) (layer "F.Cu") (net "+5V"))
 (segment (start 123 75.75) (end 126.2875 75.75) (width 0.6) (layer "F.Cu") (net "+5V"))
 (segment (start 127.25 78.25) (end 131.5 78.25) (width 0.6) (layer "F.Cu") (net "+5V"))
 (segment (start 124.7 63.65) (end 148 63.65) (width 0.6) (layer "F.Cu") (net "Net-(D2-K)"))
 (segment (start 148 69.25) (end 148 63.65) (width 0.6) (layer "F.Cu") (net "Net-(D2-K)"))
 (segment (start 120.25 56.7) (end 120.25 59.2) (width 0.6) (layer "F.Cu") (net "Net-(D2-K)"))
 (segment (start 120.25 59.2) (end 124.7 63.65) (width 0.6) (layer "F.Cu") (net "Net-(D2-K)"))
 (segment (start 115.75 65.5) (end 118.75 68.5) (width 0.6) (layer "F.Cu") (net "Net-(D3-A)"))
 (segment (start 115.75 56.2) (end 115.75 65.5) (width 0.6) (layer "F.Cu") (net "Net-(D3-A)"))
 (segment (start 126 72.6625) (end 126.7125 73.375) (width 0.6) (layer "F.Cu") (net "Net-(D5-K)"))
 (segment (start 126 68.25) (end 126 72.6625) (width 0.6) (layer "F.Cu") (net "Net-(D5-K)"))
 (segment (start 135.62 93.75) (end 135.62 92.63) (width 0.6) (layer "F.Cu") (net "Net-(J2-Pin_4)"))
 (segment (start 143 85.25) (end 144.25 85.25) (width 0.6) (layer "F.Cu") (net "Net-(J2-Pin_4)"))
 (segment (start 135.62 92.63) (end 143 85.25) (width 0.6) (layer "F.Cu") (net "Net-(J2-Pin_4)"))
 (segment (start 143.24 91.76) (end 143.25 91.75) (width 0.6) (layer "F.Cu") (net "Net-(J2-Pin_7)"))
 (segment (start 137.5 72.25) (end 138 72.25) (width 0.6) (layer "F.Cu") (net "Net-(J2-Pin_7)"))
 (segment (start 147.21 87.79) (end 148.75 87.79) (width 0.6) (layer "F.Cu") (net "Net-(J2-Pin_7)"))
 (segment (start 149.25 87.29) (end 148.75 87.79) (width 0.6) (layer "F.Cu") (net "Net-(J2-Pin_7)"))
 (segment (start 143.25 91.75) (end 146.75 91.75) (width 0.6) (layer "F.Cu") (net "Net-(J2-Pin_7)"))
 (segment (start 148.75 87.79) (end 151.55 87.79) (width 0.6) (layer "F.Cu") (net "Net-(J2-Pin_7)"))
 (segment (start 149.25 83.5) (end 149.25 87.29) (width 0.6) (layer "F.Cu") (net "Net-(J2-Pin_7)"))
 (segment (start 138 72.25) (end 149.25 83.5) (width 0.6) (layer "F.Cu") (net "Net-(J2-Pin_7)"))
 (segment (start 146.75 91.75) (end 146.75 88.25) (width 0.6) (layer "F.Cu") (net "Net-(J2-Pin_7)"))
 (segment (start 143.24 93.75) (end 143.24 91.76) (width 0.6) (layer "F.Cu") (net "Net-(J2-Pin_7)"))
 (segment (start 146.75 88.25) (end 147.21 87.79) (width 0.6) (layer "F.Cu") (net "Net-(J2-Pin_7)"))
 (segment (start 140.7 93.75) (end 140.7 90.435) (width 0.6) (layer "F.Cu") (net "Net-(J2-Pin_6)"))
 (segment (start 140.7 90.435) (end 143.345 87.79) (width 0.6) (layer "F.Cu") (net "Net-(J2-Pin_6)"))
 (segment (start 143.345 87.79) (end 144.25 87.79) (width 0.6) (layer "F.Cu") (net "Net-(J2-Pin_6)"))
 (segment (start 148.32 93.75) (end 151.55 90.52) (width 0.6) (layer "F.Cu") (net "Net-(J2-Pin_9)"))
 (segment (start 151.55 90.52) (end 151.55 89.06) (width 0.6) (layer "F.Cu") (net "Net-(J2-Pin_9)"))
 (segment (start 150.2 77.05) (end 150.25 77) (width 0.6) (layer "F.Cu") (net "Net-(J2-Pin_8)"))
 (segment (start 148 74.75) (end 148 71.25) (width 0.6) (layer "F.Cu") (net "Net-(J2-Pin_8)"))
 (segment (start 153 86.52) (end 151.55 86.52) (width 0.6) (layer "F.Cu") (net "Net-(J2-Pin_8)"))
 (segment (start 150.2 86.075) (end 150.2 77.05) (width 0.6) (layer "F.Cu") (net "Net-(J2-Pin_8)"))
 (segment (start 145.78 93.75) (end 148.28 96.25) (width 0.6) (layer "F.Cu") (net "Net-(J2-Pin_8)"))
 (segment (start 150.25 77) (end 148 74.75) (width 0.6) (layer "F.Cu") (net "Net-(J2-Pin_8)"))
 (segment (start 153.75 87.27) (end 153 86.52) (width 0.6) (layer "F.Cu") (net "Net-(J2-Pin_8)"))
 (segment (start 151.55 86.52) (end 150.645 86.52) (width 0.6) (layer "F.Cu") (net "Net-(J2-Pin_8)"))
 (segment (start 153.75 96.25) (end 153.75 87.27) (width 0.6) (layer "F.Cu") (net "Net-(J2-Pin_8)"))
 (segment (start 150.645 86.52) (end 150.2 86.075) (width 0.6) (layer "F.Cu") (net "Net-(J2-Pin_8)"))
 (segment (start 148.28 96.25) (end 153.75 96.25) (width 0.6) (layer "F.Cu") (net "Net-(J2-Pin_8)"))
 (segment (start 138.16 93.75) (end 138.16 91.705) (width 0.6) (layer "F.Cu") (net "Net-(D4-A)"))
 (segment (start 138.16 93.75) (end 142.16 97.75) (width 0.6) (layer "F.Cu") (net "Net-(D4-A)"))
 (segment (start 158.75 97.75) (end 161.5 95) (width 0.6) (layer "F.Cu") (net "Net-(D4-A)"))
 (segment (start 142.16 97.75) (end 158.75 97.75) (width 0.6) (layer "F.Cu") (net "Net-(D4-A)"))
 (segment (start 138.16 91.705) (end 143.345 86.52) (width 0.6) (layer "F.Cu") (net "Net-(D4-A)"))
 (segment (start 143.345 86.52) (end 144.25 86.52) (width 0.6) (layer "F.Cu") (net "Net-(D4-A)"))
 (segment (start 161.25 94.75) (end 161.25 71.15) (width 0.6) (layer "F.Cu") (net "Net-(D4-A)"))
 (segment (start 161.5 95) (end 161.25 94.75) (width 0.6) (layer "F.Cu") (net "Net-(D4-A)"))
 (segment (start 161.25 67.85) (end 161.25 62.75) (width 0.6) (layer "F.Cu") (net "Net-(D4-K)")))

